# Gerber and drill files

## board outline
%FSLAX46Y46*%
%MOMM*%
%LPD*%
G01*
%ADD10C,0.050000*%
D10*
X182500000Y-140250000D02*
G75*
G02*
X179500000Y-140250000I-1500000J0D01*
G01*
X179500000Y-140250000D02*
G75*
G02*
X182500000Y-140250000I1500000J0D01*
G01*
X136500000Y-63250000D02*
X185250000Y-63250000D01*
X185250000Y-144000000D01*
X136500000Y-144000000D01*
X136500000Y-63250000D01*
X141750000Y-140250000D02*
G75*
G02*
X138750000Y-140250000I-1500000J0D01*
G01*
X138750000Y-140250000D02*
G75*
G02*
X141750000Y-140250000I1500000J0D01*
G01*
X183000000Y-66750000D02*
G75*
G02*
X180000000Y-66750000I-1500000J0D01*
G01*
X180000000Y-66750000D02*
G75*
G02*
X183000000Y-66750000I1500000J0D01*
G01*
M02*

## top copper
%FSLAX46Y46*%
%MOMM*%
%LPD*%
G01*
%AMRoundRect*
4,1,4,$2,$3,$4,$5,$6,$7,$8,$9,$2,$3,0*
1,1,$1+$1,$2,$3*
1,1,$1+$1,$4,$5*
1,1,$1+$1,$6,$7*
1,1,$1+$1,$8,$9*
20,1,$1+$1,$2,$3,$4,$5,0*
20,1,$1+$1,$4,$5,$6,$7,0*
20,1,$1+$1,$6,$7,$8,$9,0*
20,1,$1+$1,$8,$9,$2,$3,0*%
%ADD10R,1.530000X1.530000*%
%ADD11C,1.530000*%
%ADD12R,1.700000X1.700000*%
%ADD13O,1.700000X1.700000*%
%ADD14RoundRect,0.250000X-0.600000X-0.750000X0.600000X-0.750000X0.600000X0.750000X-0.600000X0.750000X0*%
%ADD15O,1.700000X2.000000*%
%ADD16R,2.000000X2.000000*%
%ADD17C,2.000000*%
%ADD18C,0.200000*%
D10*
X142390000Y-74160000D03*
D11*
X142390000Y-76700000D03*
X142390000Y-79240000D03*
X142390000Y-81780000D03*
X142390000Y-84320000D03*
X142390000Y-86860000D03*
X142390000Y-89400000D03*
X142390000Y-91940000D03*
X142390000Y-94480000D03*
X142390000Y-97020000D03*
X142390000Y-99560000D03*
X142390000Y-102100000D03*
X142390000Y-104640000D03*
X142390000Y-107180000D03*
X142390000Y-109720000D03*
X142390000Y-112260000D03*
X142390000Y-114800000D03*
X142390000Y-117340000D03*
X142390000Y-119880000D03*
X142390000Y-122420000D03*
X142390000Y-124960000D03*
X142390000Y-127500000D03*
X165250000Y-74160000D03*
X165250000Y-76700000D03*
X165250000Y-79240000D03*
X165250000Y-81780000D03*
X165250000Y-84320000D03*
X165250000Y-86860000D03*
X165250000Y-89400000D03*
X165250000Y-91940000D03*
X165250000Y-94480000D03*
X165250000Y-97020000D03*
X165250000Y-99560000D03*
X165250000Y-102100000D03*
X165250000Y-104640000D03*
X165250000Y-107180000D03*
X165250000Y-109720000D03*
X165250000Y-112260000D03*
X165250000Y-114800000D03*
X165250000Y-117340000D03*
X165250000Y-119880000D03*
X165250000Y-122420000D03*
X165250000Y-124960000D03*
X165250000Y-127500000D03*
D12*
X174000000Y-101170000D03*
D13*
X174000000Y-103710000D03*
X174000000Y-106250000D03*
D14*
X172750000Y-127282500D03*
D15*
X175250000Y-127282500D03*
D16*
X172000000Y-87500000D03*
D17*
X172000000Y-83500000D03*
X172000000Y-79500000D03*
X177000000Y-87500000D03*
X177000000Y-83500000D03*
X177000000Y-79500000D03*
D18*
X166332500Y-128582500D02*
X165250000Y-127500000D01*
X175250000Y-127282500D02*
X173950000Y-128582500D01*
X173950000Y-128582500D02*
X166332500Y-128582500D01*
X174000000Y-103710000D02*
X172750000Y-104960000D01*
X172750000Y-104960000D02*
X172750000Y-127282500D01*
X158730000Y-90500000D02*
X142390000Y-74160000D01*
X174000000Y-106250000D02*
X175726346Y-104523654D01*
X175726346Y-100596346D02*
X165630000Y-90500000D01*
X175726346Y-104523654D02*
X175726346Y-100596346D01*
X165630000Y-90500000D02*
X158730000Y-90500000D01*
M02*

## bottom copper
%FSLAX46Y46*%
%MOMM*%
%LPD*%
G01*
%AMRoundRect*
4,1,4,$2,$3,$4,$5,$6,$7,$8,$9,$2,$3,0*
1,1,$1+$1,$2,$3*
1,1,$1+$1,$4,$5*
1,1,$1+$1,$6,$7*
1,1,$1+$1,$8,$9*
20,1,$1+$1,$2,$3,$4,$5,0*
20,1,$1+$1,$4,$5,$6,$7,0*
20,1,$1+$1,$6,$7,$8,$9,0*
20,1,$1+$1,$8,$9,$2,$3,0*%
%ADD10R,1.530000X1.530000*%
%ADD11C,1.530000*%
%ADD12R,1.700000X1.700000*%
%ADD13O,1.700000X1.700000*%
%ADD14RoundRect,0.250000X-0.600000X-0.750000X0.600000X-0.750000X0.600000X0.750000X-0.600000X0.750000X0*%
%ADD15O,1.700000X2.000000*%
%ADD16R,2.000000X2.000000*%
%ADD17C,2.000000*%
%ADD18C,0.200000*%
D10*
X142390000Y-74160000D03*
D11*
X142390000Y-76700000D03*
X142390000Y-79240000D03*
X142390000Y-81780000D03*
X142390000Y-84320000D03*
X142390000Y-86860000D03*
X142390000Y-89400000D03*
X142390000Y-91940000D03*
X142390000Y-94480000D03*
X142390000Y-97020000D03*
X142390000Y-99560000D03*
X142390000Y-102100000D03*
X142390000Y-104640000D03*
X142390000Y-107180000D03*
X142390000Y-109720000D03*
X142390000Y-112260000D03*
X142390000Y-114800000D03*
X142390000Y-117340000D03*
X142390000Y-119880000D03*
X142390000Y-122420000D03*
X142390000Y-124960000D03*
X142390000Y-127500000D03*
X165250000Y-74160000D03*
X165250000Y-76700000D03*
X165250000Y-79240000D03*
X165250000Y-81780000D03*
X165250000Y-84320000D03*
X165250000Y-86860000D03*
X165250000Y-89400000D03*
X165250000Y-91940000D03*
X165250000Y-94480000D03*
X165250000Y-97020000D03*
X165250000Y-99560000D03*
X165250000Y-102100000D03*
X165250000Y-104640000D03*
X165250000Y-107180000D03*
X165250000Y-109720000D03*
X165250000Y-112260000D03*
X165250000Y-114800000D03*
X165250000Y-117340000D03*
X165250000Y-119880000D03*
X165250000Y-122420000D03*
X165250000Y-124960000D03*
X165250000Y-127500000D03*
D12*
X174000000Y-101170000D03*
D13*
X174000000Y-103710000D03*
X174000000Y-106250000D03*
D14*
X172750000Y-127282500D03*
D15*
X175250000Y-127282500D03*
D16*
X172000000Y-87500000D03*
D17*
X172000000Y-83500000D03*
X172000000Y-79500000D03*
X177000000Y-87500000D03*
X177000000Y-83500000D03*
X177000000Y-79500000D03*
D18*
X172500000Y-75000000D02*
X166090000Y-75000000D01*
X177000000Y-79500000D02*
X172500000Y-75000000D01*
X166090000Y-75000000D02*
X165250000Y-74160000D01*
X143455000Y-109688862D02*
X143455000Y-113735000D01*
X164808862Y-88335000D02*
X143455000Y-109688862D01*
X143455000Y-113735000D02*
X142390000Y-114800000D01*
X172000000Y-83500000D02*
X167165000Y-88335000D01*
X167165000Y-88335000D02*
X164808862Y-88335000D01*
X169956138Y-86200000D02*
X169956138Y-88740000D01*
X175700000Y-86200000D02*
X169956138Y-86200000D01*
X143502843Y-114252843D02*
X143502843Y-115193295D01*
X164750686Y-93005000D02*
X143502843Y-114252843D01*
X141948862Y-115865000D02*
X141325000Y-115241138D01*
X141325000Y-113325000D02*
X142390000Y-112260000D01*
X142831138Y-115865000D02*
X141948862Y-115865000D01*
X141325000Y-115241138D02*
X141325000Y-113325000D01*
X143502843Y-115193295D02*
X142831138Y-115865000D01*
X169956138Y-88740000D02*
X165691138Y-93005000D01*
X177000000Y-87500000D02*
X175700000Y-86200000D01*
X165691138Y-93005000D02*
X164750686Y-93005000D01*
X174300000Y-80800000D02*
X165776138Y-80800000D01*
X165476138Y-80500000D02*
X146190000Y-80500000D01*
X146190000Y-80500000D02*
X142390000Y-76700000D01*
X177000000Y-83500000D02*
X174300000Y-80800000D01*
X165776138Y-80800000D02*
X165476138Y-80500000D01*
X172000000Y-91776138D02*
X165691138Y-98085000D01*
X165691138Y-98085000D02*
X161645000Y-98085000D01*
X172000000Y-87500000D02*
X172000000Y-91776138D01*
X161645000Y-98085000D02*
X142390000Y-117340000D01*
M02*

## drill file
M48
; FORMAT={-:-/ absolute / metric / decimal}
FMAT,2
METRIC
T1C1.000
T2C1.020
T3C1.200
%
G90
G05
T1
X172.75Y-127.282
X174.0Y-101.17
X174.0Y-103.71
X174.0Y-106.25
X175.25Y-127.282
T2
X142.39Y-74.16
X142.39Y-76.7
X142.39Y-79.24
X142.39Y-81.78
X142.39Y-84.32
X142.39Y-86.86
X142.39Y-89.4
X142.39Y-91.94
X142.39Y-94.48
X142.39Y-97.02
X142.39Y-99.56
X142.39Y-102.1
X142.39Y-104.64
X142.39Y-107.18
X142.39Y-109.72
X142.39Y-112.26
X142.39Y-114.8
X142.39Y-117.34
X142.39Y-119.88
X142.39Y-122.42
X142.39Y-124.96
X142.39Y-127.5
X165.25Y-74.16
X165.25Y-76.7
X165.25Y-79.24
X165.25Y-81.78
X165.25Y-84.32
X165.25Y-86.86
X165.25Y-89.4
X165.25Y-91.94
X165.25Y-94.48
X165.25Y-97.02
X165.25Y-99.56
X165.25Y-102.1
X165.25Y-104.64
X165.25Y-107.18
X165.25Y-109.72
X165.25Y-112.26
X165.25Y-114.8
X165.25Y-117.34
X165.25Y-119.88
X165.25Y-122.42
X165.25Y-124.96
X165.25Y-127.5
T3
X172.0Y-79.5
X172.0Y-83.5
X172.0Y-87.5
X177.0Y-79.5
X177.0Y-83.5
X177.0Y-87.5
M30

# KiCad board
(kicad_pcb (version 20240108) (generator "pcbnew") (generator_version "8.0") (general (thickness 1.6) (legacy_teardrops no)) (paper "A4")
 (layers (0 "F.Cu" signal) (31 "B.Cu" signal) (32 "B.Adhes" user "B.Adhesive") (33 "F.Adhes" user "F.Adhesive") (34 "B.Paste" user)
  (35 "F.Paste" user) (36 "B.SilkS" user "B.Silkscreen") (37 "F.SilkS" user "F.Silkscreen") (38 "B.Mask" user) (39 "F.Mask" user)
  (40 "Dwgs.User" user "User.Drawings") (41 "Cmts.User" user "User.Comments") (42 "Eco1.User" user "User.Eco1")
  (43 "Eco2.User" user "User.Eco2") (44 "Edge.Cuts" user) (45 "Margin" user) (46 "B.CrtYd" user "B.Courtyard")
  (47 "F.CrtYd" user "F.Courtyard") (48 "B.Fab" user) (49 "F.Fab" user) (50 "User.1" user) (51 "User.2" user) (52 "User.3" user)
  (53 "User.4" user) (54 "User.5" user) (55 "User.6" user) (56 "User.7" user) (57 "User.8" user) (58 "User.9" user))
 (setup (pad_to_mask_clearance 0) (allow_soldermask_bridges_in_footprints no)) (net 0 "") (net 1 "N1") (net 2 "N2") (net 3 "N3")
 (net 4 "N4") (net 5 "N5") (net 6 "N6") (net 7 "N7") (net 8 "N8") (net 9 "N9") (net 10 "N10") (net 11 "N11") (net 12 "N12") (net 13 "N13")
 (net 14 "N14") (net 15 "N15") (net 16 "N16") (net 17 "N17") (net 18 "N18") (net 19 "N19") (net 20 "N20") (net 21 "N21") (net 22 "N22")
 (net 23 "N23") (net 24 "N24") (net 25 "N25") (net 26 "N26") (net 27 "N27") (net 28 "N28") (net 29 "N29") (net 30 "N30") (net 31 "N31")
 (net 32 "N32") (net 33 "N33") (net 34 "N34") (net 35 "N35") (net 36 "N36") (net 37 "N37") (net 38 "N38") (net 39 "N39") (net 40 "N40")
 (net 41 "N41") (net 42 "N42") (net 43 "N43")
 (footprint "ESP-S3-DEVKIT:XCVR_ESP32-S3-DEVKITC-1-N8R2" (layer "F.Cu") (at 153.82 104.13)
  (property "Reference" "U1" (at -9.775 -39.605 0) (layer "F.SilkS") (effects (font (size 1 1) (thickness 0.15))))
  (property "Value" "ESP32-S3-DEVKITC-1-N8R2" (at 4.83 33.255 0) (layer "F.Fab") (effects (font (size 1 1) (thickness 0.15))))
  (pad "J1_1" thru_hole rect (at -11.43 -29.97) (size 1.53 1.53) (drill 1.02) (layers "*.Cu" "*.Mask") (remove_unused_layers no)
   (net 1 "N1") (solder_mask_margin 0.102))
  (pad "J1_2" thru_hole circle (at -11.43 -27.43) (size 1.53 1.53) (drill 1.02) (layers "*.Cu" "*.Mask") (remove_unused_layers no)
   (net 1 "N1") (solder_mask_margin 0.102))
  (pad "J1_3" thru_hole circle (at -11.43 -24.89) (size 1.53 1.53) (drill 1.02) (layers "*.Cu" "*.Mask") (remove_unused_layers no)
   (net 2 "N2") (solder_mask_margin 0.102))
  (pad "J1_4" thru_hole circle (at -11.43 -22.35) (size 1.53 1.53) (drill 1.02) (layers "*.Cu" "*.Mask") (remove_unused_layers no)
   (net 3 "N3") (solder_mask_margin 0.102))
  (pad "J1_5" thru_hole circle (at -11.43 -19.81) (size 1.53 1.53) (drill 1.02) (layers "*.Cu" "*.Mask") (remove_unused_layers no)
   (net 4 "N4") (solder_mask_margin 0.102))
  (pad "J1_6" thru_hole circle (at -11.43 -17.27) (size 1.53 1.53) (drill 1.02) (layers "*.Cu" "*.Mask") (remove_unused_layers no)
   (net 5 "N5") (solder_mask_margin 0.102))
  (pad "J1_7" thru_hole circle (at -11.43 -14.73) (size 1.53 1.53) (drill 1.02) (layers "*.Cu" "*.Mask") (remove_unused_layers no)
   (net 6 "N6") (solder_mask_margin 0.102))
  (pad "J1_8" thru_hole circle (at -11.43 -12.19) (size 1.53 1.53) (drill 1.02) (layers "*.Cu" "*.Mask") (remove_unused_layers no)
   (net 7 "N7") (solder_mask_margin 0.102))
  (pad "J1_9" thru_hole circle (at -11.43 -9.65) (size 1.53 1.53) (drill 1.02) (layers "*.Cu" "*.Mask") (remove_unused_layers no)
   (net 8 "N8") (solder_mask_margin 0.102))
  (pad "J1_10" thru_hole circle (at -11.43 -7.11) (size 1.53 1.53) (drill 1.02) (layers "*.Cu" "*.Mask") (remove_unused_layers no)
   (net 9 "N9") (solder_mask_margin 0.102))
  (pad "J1_11" thru_hole circle (at -11.43 -4.57) (size 1.53 1.53) (drill 1.02) (layers "*.Cu" "*.Mask") (remove_unused_layers no)
   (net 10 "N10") (solder_mask_margin 0.102))
  (pad "J1_12" thru_hole circle (at -11.43 -2.03) (size 1.53 1.53) (drill 1.02) (layers "*.Cu" "*.Mask") (remove_unused_layers no)
   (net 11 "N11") (solder_mask_margin 0.102))
  (pad "J1_13" thru_hole circle (at -11.43 0.51) (size 1.53 1.53) (drill 1.02) (layers "*.Cu" "*.Mask") (remove_unused_layers no)
   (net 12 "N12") (solder_mask_margin 0.102))
  (pad "J1_14" thru_hole circle (at -11.43 3.05) (size 1.53 1.53) (drill 1.02) (layers "*.Cu" "*.Mask") (remove_unused_layers no)
   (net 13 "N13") (solder_mask_margin 0.102))
  (pad "J1_15" thru_hole circle (at -11.43 5.59) (size 1.53 1.53) (drill 1.02) (layers "*.Cu" "*.Mask") (remove_unused_layers no)
   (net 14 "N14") (solder_mask_margin 0.102))
  (pad "J1_16" thru_hole circle (at -11.43 8.13) (size 1.53 1.53) (drill 1.02) (layers "*.Cu" "*.Mask") (remove_unused_layers no)
   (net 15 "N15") (solder_mask_margin 0.102))
  (pad "J1_17" thru_hole circle (at -11.43 10.67) (size 1.53 1.53) (drill 1.02) (layers "*.Cu" "*.Mask") (remove_unused_layers no)
   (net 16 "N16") (solder_mask_margin 0.102))
  (pad "J1_18" thru_hole circle (at -11.43 13.21) (size 1.53 1.53) (drill 1.02) (layers "*.Cu" "*.Mask") (remove_unused_layers no)
   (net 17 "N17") (solder_mask_margin 0.102))
  (pad "J1_19" thru_hole circle (at -11.43 15.75) (size 1.53 1.53) (drill 1.02) (layers "*.Cu" "*.Mask") (remove_unused_layers no)
   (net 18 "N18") (solder_mask_margin 0.102))
  (pad "J1_20" thru_hole circle (at -11.43 18.29) (size 1.53 1.53) (drill 1.02) (layers "*.Cu" "*.Mask") (remove_unused_layers no)
   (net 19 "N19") (solder_mask_margin 0.102))
  (pad "J1_21" thru_hole circle (at -11.43 20.83) (size 1.53 1.53) (drill 1.02) (layers "*.Cu" "*.Mask") (remove_unused_layers no)
   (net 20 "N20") (solder_mask_margin 0.102))
  (pad "J1_22" thru_hole circle (at -11.43 23.37) (size 1.53 1.53) (drill 1.02) (layers "*.Cu" "*.Mask") (remove_unused_layers no)
   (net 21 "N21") (solder_mask_margin 0.102))
  (pad "J3_1" thru_hole circle (at 11.43 -29.97) (size 1.53 1.53) (drill 1.02) (layers "*.Cu" "*.Mask") (remove_unused_layers no)
   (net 21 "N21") (solder_mask_margin 0.102))
  (pad "J3_2" thru_hole circle (at 11.43 -27.43) (size 1.53 1.53) (drill 1.02) (layers "*.Cu" "*.Mask") (remove_unused_layers no)
   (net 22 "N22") (solder_mask_margin 0.102))
  (pad "J3_3" thru_hole circle (at 11.43 -24.89) (size 1.53 1.53) (drill 1.02) (layers "*.Cu" "*.Mask") (remove_unused_layers no)
   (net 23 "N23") (solder_mask_margin 0.102))
  (pad "J3_4" thru_hole circle (at 11.43 -22.35) (size 1.53 1.53) (drill 1.02) (layers "*.Cu" "*.Mask") (remove_unused_layers no)
   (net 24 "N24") (solder_mask_margin 0.102))
  (pad "J3_5" thru_hole circle (at 11.43 -19.81) (size 1.53 1.53) (drill 1.02) (layers "*.Cu" "*.Mask") (remove_unused_layers no)
   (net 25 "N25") (solder_mask_margin 0.102))
  (pad "J3_6" thru_hole circle (at 11.43 -17.27) (size 1.53 1.53) (drill 1.02) (layers "*.Cu" "*.Mask") (remove_unused_layers no)
   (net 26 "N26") (solder_mask_margin 0.102))
  (pad "J3_7" thru_hole circle (at 11.43 -14.73) (size 1.53 1.53) (drill 1.02) (layers "*.Cu" "*.Mask") (remove_unused_layers no)
   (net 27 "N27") (solder_mask_margin 0.102))
  (pad "J3_8" thru_hole circle (at 11.43 -12.19) (size 1.53 1.53) (drill 1.02) (layers "*.Cu" "*.Mask") (remove_unused_layers no)
   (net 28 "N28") (solder_mask_margin 0.102))
  (pad "J3_9" thru_hole circle (at 11.43 -9.65) (size 1.53 1.53) (drill 1.02) (layers "*.Cu" "*.Mask") (remove_unused_layers no)
   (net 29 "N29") (solder_mask_margin 0.102))
  (pad "J3_10" thru_hole circle (at 11.43 -7.11) (size 1.53 1.53) (drill 1.02) (layers "*.Cu" "*.Mask") (remove_unused_layers no)
   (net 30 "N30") (solder_mask_margin 0.102))
  (pad "J3_11" thru_hole circle (at 11.43 -4.57) (size 1.53 1.53) (drill 1.02) (layers "*.Cu" "*.Mask") (remove_unused_layers no)
   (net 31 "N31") (solder_mask_margin 0.102))
  (pad "J3_12" thru_hole circle (at 11.43 -2.03) (size 1.53 1.53) (drill 1.02) (layers "*.Cu" "*.Mask") (remove_unused_layers no)
   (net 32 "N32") (solder_mask_margin 0.102))
  (pad "J3_13" thru_hole circle (at 11.43 0.51) (size 1.53 1.53) (drill 1.02) (layers "*.Cu" "*.Mask") (remove_unused_layers no)
   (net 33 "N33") (solder_mask_margin 0.102))
  (pad "J3_14" thru_hole circle (at 11.43 3.05) (size 1.53 1.53) (drill 1.02) (layers "*.Cu" "*.Mask") (remove_unused_layers no)
   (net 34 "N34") (solder_mask_margin 0.102))
  (pad "J3_15" thru_hole circle (at 11.43 5.59) (size 1.53 1.53) (drill 1.02) (layers "*.Cu" "*.Mask") (remove_unused_layers no)
   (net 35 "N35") (solder_mask_margin 0.102))
  (pad "J3_16" thru_hole circle (at 11.43 8.13) (size 1.53 1.53) (drill 1.02) (layers "*.Cu" "*.Mask") (remove_unused_layers no)
   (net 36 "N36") (solder_mask_margin 0.102))
  (pad "J3_17" thru_hole circle (at 11.43 10.67) (size 1.53 1.53) (drill 1.02) (layers "*.Cu" "*.Mask") (remove_unused_layers no)
   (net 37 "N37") (solder_mask_margin 0.102))
  (pad "J3_18" thru_hole circle (at 11.43 13.21) (size 1.53 1.53) (drill 1.02) (layers "*.Cu" "*.Mask") (remove_unused_layers no)
   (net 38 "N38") (solder_mask_margin 0.102))
  (pad "J3_19" thru_hole circle (at 11.43 15.75) (size 1.53 1.53) (drill 1.02) (layers "*.Cu" "*.Mask") (remove_unused_layers no)
   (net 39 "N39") (solder_mask_margin 0.102))
  (pad "J3_20" thru_hole circle (at 11.43 18.29) (size 1.53 1.53) (drill 1.02) (layers "*.Cu" "*.Mask") (remove_unused_layers no)
   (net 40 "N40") (solder_mask_margin 0.102))
  (pad "J3_21" thru_hole circle (at 11.43 20.83) (size 1.53 1.53) (drill 1.02) (layers "*.Cu" "*.Mask") (remove_unused_layers no)
   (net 21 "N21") (solder_mask_margin 0.102))
  (pad "J3_22" thru_hole circle (at 11.43 23.37) (size 1.53 1.53) (drill 1.02) (layers "*.Cu" "*.Mask") (remove_unused_layers no)
   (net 21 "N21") (solder_mask_margin 0.102)))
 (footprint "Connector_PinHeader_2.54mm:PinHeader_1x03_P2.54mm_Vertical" (layer "F.Cu") (at 174 101.17)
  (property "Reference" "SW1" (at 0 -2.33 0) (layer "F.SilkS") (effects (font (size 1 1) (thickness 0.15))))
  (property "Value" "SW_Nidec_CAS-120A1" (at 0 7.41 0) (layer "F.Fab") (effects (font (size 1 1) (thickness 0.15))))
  (pad "1" thru_hole rect (at 0 0) (size 1.7 1.7) (drill 1) (layers "*.Cu" "*.Mask") (remove_unused_layers no) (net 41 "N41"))
  (pad "2" thru_hole oval (at 0 2.54) (size 1.7 1.7) (drill 1) (layers "*.Cu" "*.Mask") (remove_unused_layers no) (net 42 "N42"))
  (pad "3" thru_hole oval (at 0 5.08) (size 1.7 1.7) (drill 1) (layers "*.Cu" "*.Mask") (remove_unused_layers no) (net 1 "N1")))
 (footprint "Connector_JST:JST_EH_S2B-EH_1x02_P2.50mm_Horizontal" (layer "F.Cu") (at 172.75 127.2825)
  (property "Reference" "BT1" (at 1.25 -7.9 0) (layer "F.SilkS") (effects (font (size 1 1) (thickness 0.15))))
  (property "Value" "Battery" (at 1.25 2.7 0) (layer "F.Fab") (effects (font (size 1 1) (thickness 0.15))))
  (pad "1" thru_hole roundrect (at 0 0) (size 1.7 2) (drill 1) (layers "*.Cu" "*.Mask") (remove_unused_layers no)
   (roundrect_rratio 0.147059) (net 42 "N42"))
  (pad "2" thru_hole oval (at 2.5 0) (size 1.7 2) (drill 1) (layers "*.Cu" "*.Mask") (remove_unused_layers no) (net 21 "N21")))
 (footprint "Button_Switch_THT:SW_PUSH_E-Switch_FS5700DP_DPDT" (layer "F.Cu") (at 172 87.5 90)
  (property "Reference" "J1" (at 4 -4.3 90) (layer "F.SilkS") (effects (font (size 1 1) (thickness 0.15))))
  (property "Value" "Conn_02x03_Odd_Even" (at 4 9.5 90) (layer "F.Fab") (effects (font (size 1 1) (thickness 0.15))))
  (pad "1" thru_hole rect (at 0 0 90) (size 2 2) (drill 1.2) (layers "*.Cu" "*.Mask") (remove_unused_layers no) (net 17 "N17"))
  (pad "2" thru_hole circle (at 4 0 90) (size 2 2) (drill 1.2) (layers "*.Cu" "*.Mask") (remove_unused_layers no) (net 16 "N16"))
  (pad "3" thru_hole circle (at 8 0 90) (size 2 2) (drill 1.2) (layers "*.Cu" "*.Mask") (remove_unused_layers no) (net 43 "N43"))
  (pad "4" thru_hole circle (at 0 5 90) (size 2 2) (drill 1.2) (layers "*.Cu" "*.Mask") (remove_unused_layers no) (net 15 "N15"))
  (pad "5" thru_hole circle (at 4 5 90) (size 2 2) (drill 1.2) (layers "*.Cu" "*.Mask") (remove_unused_layers no) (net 1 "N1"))
  (pad "6" thru_hole circle (at 8 5 90) (size 2 2) (drill 1.2) (layers "*.Cu" "*.Mask") (remove_unused_layers no) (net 21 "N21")))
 (gr_circle (center 181 140.25) (end 182.5 140.25) (stroke (width 0.05) (type default)) (fill none) (layer "Edge.Cuts"))
 (gr_rect (start 136.5 63.25) (end 185.25 144) (stroke (width 0.05) (type default)) (fill none) (layer "Edge.Cuts"))
 (gr_circle (center 140.25 140.25) (end 141.75 140.25) (stroke (width 0.05) (type default)) (fill none) (layer "Edge.Cuts"))
 (gr_circle (center 181.5 66.75) (end 183 66.75) (stroke (width 0.05) (type default)) (fill none) (layer "Edge.Cuts"))
 (segment (start 166.3325 128.5825) (end 165.25 127.5) (width 0.2) (layer "F.Cu") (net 21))
 (segment (start 175.25 127.2825) (end 173.95 128.5825) (width 0.2) (layer "F.Cu") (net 21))
 (segment (start 173.95 128.5825) (end 166.3325 128.5825) (width 0.2) (layer "F.Cu") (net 21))
 (segment (start 172.5 75) (end 166.09 75) (width 0.2) (layer "B.Cu") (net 21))
 (segment (start 177 79.5) (end 172.5 75) (width 0.2) (layer "B.Cu") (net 21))
 (segment (start 166.09 75) (end 165.25 74.16) (width 0.2) (layer "B.Cu") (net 21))
 (segment (start 174 103.71) (end 172.75 104.96) (width 0.2) (layer "F.Cu") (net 42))
 (segment (start 172.75 104.96) (end 172.75 127.2825) (width 0.2) (layer "F.Cu") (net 42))
 (segment (start 143.455 109.688862) (end 143.455 113.735) (width 0.2) (layer "B.Cu") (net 16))
 (segment (start 164.808862 88.335) (end 143.455 109.688862) (width 0.2) (layer "B.Cu") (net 16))
 (segment (start 143.455 113.735) (end 142.39 114.8) (width 0.2) (layer "B.Cu") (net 16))
 (segment (start 172 83.5) (end 167.165 88.335) (width 0.2) (layer "B.Cu") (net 16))
 (segment (start 167.165 88.335) (end 164.808862 88.335) (width 0.2) (layer "B.Cu") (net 16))
 (segment (start 169.956138 86.2) (end 169.956138 88.74) (width 0.2) (layer "B.Cu") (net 15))
 (segment (start 175.7 86.2) (end 169.956138 86.2) (width 0.2) (layer "B.Cu") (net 15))
 (segment (start 143.502843 114.252843) (end 143.502843 115.193295) (width 0.2) (layer "B.Cu") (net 15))
 (segment (start 164.750686 93.005) (end 143.502843 114.252843) (width 0.2) (layer "B.Cu") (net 15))
 (segment (start 141.948862 115.865) (end 141.325 115.241138) (width 0.2) (layer "B.Cu") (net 15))
 (segment (start 141.325 113.325) (end 142.39 112.26) (width 0.2) (layer "B.Cu") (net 15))
 (segment (start 142.831138 115.865) (end 141.948862 115.865) (width 0.2) (layer "B.Cu") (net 15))
 (segment (start 141.325 115.241138) (end 141.325 113.325) (width 0.2) (layer "B.Cu") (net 15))
 (segment (start 143.502843 115.193295) (end 142.831138 115.865) (width 0.2) (layer "B.Cu") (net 15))
 (segment (start 169.956138 88.74) (end 165.691138 93.005) (width 0.2) (layer "B.Cu") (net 15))
 (segment (start 177 87.5) (end 175.7 86.2) (width 0.2) (layer "B.Cu") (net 15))
 (segment (start 165.691138 93.005) (end 164.750686 93.005) (width 0.2) (layer "B.Cu") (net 15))
 (segment (start 158.73 90.5) (end 142.39 74.16) (width 0.2) (layer "F.Cu") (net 1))
 (segment (start 174 106.25) (end 175.726346 104.523654) (width 0.2) (layer "F.Cu") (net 1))
 (segment (start 175.726346 100.596346) (end 165.63 90.5) (width 0.2) (layer "F.Cu") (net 1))
 (segment (start 175.726346 104.523654) (end 175.726346 100.596346) (width 0.2) (layer "F.Cu") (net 1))
 (segment (start 165.63 90.5) (end 158.73 90.5) (width 0.2) (layer "F.Cu") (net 1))
 (segment (start 174.3 80.8) (end 165.776138 80.8) (width 0.2) (layer "B.Cu") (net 1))
 (segment (start 165.476138 80.5) (end 146.19 80.5) (width 0.2) (layer "B.Cu") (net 1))
 (segment (start 146.19 80.5) (end 142.39 76.7) (width 0.2) (layer "B.Cu") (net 1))
 (segment (start 177 83.5) (end 174.3 80.8) (width 0.2) (layer "B.Cu") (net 1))
 (segment (start 165.776138 80.8) (end 165.476138 80.5) (width 0.2) (layer "B.Cu") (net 1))
 (segment (start 172 91.776138) (end 165.691138 98.085) (width 0.2) (layer "B.Cu") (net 17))
 (segment (start 165.691138 98.085) (end 161.645 98.085) (width 0.2) (layer "B.Cu") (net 17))
 (segment (start 172 87.5) (end 172 91.776138) (width 0.2) (layer "B.Cu") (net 17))
 (segment (start 161.645 98.085) (end 142.39 117.34) (width 0.2) (layer "B.Cu") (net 17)))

